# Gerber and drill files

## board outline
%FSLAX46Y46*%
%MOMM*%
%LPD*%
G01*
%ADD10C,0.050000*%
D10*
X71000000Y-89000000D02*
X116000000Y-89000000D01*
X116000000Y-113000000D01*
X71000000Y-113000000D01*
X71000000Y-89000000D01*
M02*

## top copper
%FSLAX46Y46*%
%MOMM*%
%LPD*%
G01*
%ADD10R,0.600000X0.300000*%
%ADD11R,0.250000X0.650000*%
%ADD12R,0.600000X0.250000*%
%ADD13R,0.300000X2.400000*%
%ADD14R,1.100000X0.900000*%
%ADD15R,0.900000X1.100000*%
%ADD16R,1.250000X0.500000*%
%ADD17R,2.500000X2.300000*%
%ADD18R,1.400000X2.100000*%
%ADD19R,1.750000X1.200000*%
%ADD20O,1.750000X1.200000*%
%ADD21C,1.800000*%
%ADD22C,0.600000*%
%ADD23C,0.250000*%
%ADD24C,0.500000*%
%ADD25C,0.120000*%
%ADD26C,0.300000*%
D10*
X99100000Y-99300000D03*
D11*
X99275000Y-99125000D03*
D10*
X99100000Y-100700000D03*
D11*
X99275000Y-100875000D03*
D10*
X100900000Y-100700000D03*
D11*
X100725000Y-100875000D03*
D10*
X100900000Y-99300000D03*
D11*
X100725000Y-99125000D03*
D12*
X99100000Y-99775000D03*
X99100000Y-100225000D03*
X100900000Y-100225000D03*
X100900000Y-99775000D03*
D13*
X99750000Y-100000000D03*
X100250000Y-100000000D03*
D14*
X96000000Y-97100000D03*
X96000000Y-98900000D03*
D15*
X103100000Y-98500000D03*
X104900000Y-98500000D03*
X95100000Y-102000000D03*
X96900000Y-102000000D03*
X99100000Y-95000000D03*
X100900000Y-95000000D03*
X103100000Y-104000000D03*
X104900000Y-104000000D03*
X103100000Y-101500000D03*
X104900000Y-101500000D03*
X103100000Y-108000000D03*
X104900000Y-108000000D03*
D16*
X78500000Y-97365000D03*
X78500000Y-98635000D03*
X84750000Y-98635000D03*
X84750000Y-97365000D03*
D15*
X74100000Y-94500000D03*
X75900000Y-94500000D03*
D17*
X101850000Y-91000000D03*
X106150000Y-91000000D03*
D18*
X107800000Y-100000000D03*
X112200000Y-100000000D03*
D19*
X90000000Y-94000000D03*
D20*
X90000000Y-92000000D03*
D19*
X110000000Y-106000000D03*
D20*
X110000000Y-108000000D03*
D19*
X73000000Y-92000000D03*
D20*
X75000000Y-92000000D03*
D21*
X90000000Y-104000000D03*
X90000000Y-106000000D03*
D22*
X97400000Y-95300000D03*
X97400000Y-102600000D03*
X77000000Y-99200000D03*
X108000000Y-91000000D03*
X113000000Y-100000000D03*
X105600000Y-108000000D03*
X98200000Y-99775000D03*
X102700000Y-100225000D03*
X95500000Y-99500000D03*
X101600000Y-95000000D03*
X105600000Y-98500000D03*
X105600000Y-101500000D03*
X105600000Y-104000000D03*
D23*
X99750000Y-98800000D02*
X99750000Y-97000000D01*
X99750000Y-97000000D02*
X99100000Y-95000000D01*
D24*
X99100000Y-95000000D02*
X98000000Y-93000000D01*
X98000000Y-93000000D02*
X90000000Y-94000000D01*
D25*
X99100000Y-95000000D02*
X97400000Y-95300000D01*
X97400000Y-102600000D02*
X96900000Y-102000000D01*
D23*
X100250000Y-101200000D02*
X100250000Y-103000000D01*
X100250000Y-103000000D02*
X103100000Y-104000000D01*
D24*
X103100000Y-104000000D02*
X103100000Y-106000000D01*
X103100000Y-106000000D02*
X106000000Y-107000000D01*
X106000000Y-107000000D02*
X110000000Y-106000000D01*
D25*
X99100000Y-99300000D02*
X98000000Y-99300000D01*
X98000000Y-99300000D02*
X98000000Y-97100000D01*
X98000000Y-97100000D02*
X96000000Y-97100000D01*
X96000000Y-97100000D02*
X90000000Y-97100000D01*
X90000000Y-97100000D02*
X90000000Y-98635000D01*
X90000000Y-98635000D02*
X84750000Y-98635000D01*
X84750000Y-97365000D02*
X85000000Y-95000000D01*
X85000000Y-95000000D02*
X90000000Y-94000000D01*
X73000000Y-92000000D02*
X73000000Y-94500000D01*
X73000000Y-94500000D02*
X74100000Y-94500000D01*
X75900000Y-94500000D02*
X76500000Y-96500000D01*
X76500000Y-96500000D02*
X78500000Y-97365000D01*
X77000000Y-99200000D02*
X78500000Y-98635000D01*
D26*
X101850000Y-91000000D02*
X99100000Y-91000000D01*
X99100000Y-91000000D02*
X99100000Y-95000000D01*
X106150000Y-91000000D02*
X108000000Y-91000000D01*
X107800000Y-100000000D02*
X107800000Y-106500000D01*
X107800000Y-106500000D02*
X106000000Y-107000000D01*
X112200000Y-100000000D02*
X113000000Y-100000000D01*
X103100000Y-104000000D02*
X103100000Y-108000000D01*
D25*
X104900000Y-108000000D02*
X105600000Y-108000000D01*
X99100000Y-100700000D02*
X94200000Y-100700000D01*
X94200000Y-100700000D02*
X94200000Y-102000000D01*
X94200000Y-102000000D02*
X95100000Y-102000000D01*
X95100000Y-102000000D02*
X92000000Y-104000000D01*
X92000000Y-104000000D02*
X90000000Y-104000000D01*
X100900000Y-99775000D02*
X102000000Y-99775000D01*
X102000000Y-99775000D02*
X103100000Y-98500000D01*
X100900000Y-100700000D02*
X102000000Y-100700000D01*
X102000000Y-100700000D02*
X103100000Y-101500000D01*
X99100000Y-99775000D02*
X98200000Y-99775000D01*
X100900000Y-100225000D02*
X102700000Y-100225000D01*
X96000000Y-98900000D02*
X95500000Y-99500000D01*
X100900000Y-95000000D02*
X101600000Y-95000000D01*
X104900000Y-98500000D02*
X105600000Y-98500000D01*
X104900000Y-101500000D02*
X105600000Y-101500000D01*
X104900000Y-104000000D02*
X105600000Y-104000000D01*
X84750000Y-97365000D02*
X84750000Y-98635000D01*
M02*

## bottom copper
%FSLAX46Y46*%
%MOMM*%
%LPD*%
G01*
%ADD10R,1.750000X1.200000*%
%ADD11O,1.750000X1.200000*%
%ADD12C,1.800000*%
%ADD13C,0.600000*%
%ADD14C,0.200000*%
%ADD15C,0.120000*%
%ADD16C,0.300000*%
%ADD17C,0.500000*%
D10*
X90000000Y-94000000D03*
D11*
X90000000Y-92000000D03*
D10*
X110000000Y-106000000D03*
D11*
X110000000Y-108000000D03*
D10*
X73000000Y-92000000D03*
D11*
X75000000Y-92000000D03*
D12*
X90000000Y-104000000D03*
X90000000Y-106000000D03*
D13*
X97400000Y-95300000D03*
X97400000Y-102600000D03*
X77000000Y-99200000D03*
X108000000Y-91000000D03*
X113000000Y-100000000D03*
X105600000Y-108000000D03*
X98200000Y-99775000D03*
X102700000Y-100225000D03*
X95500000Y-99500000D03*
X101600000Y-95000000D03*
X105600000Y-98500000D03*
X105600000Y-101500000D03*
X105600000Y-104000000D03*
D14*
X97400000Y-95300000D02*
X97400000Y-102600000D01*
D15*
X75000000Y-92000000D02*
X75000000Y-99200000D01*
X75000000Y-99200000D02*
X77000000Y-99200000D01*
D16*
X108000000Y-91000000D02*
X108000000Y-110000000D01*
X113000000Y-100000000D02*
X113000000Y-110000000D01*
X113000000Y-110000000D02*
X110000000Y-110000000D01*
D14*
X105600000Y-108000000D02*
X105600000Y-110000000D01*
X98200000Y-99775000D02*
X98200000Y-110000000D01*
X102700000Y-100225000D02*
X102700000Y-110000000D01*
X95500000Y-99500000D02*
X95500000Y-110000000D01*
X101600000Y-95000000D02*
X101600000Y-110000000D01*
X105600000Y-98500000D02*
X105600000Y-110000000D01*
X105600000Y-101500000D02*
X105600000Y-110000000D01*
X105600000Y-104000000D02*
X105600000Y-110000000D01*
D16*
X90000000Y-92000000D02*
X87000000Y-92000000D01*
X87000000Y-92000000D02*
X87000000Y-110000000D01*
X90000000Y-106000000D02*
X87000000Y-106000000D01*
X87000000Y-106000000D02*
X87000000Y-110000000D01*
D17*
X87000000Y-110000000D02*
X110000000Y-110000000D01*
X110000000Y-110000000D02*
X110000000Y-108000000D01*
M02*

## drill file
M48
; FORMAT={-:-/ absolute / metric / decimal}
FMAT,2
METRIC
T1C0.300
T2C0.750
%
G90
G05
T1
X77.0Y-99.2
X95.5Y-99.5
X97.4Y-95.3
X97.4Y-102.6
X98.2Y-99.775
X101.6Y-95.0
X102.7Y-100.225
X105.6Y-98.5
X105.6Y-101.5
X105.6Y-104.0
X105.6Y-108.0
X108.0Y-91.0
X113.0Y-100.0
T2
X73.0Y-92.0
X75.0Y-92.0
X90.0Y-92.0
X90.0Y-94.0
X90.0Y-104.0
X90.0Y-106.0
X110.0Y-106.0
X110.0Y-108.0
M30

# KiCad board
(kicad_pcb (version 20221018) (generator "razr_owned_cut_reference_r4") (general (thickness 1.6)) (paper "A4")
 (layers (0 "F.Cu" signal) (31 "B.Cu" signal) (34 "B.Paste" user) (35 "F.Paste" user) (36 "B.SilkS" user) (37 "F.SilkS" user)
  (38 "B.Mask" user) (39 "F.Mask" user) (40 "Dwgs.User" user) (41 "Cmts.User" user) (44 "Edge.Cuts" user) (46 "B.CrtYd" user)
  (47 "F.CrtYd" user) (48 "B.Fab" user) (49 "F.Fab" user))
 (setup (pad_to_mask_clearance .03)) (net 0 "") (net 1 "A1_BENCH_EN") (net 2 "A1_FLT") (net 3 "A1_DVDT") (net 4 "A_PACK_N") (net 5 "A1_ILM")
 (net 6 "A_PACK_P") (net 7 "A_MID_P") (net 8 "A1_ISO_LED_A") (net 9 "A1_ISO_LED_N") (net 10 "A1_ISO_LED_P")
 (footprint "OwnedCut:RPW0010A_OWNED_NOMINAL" (layer "F.Cu") (at 100 100)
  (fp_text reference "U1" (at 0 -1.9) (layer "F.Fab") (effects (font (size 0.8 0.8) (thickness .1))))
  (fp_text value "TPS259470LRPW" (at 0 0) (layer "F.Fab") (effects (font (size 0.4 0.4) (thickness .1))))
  (pad "1" smd rect (at -0.9 -0.7) (size 0.6 0.3) (layers "F.Cu" "F.Paste" "F.Mask") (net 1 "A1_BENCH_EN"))
  (pad "1" smd rect (at -0.725 -0.875) (size 0.25 0.65) (layers "F.Cu" "F.Paste" "F.Mask") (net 1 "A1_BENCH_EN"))
  (pad "4" smd rect (at -0.9 0.7) (size 0.6 0.3) (layers "F.Cu" "F.Paste" "F.Mask") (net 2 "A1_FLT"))
  (pad "4" smd rect (at -0.725 0.875) (size 0.25 0.65) (layers "F.Cu" "F.Paste" "F.Mask") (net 2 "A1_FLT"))
  (pad "7" smd rect (at 0.9 0.7) (size 0.6 0.3) (layers "F.Cu" "F.Paste" "F.Mask") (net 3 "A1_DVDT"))
  (pad "7" smd rect (at 0.725 0.875) (size 0.25 0.65) (layers "F.Cu" "F.Paste" "F.Mask") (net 3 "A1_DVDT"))
  (pad "10" smd rect (at 0.9 -0.7) (size 0.6 0.3) (layers "F.Cu" "F.Paste" "F.Mask"))
  (pad "10" smd rect (at 0.725 -0.875) (size 0.25 0.65) (layers "F.Cu" "F.Paste" "F.Mask"))
  (pad "2" smd rect (at -0.9 -0.225) (size 0.6 0.25) (layers "F.Cu" "F.Paste" "F.Mask") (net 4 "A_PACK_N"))
  (pad "3" smd rect (at -0.9 0.225) (size 0.6 0.25) (layers "F.Cu" "F.Paste" "F.Mask"))
  (pad "8" smd rect (at 0.9 0.225) (size 0.6 0.25) (layers "F.Cu" "F.Paste" "F.Mask") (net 4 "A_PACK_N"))
  (pad "9" smd rect (at 0.9 -0.225) (size 0.6 0.25) (layers "F.Cu" "F.Paste" "F.Mask") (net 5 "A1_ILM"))
  (pad "5" smd rect (at -0.25 0) (size 0.3 2.4) (layers "F.Cu" "F.Paste" "F.Mask") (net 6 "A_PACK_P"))
  (pad "6" smd rect (at 0.25 0) (size 0.3 2.4) (layers "F.Cu" "F.Paste" "F.Mask") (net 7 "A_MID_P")))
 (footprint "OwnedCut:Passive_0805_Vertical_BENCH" (layer "F.Cu") (at 96 98)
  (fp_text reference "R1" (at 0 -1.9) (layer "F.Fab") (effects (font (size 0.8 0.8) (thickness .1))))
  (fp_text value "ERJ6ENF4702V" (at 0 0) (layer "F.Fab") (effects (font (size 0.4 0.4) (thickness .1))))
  (pad "1" smd rect (at 0 -0.9) (size 1.1 0.9) (layers "F.Cu" "F.Paste" "F.Mask") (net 1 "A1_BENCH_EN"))
  (pad "2" smd rect (at 0 0.9) (size 1.1 0.9) (layers "F.Cu" "F.Paste" "F.Mask") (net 4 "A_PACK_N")))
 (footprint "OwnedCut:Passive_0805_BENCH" (layer "F.Cu") (at 104 98.5)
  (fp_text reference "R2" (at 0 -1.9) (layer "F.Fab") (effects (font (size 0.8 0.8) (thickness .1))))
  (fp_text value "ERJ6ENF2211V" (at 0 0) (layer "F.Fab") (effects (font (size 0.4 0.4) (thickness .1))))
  (pad "1" smd rect (at -0.9 0) (size 0.9 1.1) (layers "F.Cu" "F.Paste" "F.Mask") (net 5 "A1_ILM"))
  (pad "2" smd rect (at 0.9 0) (size 0.9 1.1) (layers "F.Cu" "F.Paste" "F.Mask") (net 4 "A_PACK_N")))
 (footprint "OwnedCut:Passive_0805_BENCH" (layer "F.Cu") (at 96 102)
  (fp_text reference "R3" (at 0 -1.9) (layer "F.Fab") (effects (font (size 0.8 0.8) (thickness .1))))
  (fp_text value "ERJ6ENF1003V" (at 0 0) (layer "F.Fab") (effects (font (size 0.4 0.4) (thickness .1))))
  (pad "1" smd rect (at -0.9 0) (size 0.9 1.1) (layers "F.Cu" "F.Paste" "F.Mask") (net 2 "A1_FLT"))
  (pad "2" smd rect (at 0.9 0) (size 0.9 1.1) (layers "F.Cu" "F.Paste" "F.Mask") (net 6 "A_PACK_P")))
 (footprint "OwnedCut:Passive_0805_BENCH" (layer "F.Cu") (at 100 95)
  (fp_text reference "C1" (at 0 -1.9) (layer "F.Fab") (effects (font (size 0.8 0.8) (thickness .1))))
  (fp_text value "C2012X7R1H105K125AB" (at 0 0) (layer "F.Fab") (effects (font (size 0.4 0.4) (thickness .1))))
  (pad "1" smd rect (at -0.9 0) (size 0.9 1.1) (layers "F.Cu" "F.Paste" "F.Mask") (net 6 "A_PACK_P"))
  (pad "2" smd rect (at 0.9 0) (size 0.9 1.1) (layers "F.Cu" "F.Paste" "F.Mask") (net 4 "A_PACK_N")))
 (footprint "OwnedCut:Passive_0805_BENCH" (layer "F.Cu") (at 104 104)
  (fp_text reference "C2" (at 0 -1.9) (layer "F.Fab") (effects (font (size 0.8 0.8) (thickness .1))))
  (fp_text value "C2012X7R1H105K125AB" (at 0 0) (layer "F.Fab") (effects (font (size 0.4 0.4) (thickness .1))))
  (pad "1" smd rect (at -0.9 0) (size 0.9 1.1) (layers "F.Cu" "F.Paste" "F.Mask") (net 7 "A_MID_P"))
  (pad "2" smd rect (at 0.9 0) (size 0.9 1.1) (layers "F.Cu" "F.Paste" "F.Mask") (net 4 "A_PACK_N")))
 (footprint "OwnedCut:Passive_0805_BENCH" (layer "F.Cu") (at 104 101.5)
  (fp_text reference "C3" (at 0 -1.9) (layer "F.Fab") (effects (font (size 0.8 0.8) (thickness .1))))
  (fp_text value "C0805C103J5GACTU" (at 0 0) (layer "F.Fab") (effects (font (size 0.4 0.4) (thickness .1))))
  (pad "1" smd rect (at -0.9 0) (size 0.9 1.1) (layers "F.Cu" "F.Paste" "F.Mask") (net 3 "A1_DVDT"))
  (pad "2" smd rect (at 0.9 0) (size 0.9 1.1) (layers "F.Cu" "F.Paste" "F.Mask") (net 4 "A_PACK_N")))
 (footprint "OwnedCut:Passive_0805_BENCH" (layer "F.Cu") (at 104 108)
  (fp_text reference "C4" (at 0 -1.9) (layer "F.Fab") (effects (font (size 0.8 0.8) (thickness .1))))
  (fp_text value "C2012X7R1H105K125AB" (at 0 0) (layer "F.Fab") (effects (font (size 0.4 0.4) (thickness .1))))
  (pad "1" smd rect (at -0.9 0) (size 0.9 1.1) (layers "F.Cu" "F.Paste" "F.Mask") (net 7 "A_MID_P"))
  (pad "2" smd rect (at 0.9 0) (size 0.9 1.1) (layers "F.Cu" "F.Paste" "F.Mask") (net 4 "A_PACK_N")))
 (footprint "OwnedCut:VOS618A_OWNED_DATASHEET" (layer "F.Cu") (at 81.625 98)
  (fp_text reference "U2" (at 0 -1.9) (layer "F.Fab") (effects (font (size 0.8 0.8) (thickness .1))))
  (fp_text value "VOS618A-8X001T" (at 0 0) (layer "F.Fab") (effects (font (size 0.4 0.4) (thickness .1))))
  (pad "1" smd rect (at -3.125 -0.635) (size 1.25 0.5) (layers "F.Cu" "F.Paste" "F.Mask") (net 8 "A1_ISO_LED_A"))
  (pad "2" smd rect (at -3.125 0.635) (size 1.25 0.5) (layers "F.Cu" "F.Paste" "F.Mask") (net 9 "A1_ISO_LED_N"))
  (pad "3" smd rect (at 3.125 0.635) (size 1.25 0.5) (layers "F.Cu" "F.Paste" "F.Mask") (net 1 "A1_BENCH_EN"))
  (pad "4" smd rect (at 3.125 -0.635) (size 1.25 0.5) (layers "F.Cu" "F.Paste" "F.Mask") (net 6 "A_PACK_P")))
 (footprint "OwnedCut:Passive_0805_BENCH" (layer "F.Cu") (at 75 94.5)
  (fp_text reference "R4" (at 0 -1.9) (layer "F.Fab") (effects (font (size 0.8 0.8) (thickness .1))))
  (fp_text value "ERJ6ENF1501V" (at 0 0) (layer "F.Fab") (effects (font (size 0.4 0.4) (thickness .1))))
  (pad "1" smd rect (at -0.9 0) (size 0.9 1.1) (layers "F.Cu" "F.Paste" "F.Mask") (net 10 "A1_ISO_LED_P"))
  (pad "2" smd rect (at 0.9 0) (size 0.9 1.1) (layers "F.Cu" "F.Paste" "F.Mask") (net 8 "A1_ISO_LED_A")))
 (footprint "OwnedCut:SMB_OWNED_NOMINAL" (layer "F.Cu") (at 104 91)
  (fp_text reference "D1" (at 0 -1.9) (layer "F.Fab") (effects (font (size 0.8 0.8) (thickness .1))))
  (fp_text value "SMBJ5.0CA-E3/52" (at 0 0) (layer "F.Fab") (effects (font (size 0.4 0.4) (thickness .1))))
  (pad "1" smd rect (at -2.15 0) (size 2.5 2.3) (layers "F.Cu" "F.Paste" "F.Mask") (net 6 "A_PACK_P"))
  (pad "2" smd rect (at 2.15 0) (size 2.5 2.3) (layers "F.Cu" "F.Paste" "F.Mask") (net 4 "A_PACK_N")))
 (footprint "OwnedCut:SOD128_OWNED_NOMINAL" (layer "F.Cu") (at 110 100)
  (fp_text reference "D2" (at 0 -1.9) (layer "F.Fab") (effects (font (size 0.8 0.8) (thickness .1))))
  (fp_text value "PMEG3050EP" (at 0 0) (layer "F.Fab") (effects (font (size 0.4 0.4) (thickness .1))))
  (pad "1" smd rect (at -2.2 0) (size 1.4 2.1) (layers "F.Cu" "F.Paste" "F.Mask") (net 7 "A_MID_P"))
  (pad "2" smd rect (at 2.2 0) (size 1.4 2.1) (layers "F.Cu" "F.Paste" "F.Mask") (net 4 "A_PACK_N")))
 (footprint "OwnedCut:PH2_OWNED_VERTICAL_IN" (layer "F.Cu") (at 90 94)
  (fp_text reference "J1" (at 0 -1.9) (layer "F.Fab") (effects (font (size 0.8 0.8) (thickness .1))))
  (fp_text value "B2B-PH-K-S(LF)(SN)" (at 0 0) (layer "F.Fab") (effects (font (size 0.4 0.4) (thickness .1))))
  (pad "1" thru_hole rect (at 0 0) (size 1.75 1.2) (drill .75) (layers "*.Cu" "*.Mask") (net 6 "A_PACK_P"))
  (pad "2" thru_hole oval (at 0 -2) (size 1.75 1.2) (drill .75) (layers "*.Cu" "*.Mask") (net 4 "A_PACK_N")))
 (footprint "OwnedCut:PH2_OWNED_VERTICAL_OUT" (layer "F.Cu") (at 110 106)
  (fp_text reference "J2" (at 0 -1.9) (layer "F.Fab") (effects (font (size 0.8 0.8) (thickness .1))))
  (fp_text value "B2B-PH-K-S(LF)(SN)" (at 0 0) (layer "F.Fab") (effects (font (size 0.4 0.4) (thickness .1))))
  (pad "1" thru_hole rect (at 0 0) (size 1.75 1.2) (drill .75) (layers "*.Cu" "*.Mask") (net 7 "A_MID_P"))
  (pad "2" thru_hole oval (at 0 2) (size 1.75 1.2) (drill .75) (layers "*.Cu" "*.Mask") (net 4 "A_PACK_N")))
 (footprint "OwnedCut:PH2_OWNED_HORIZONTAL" (layer "F.Cu") (at 73 92)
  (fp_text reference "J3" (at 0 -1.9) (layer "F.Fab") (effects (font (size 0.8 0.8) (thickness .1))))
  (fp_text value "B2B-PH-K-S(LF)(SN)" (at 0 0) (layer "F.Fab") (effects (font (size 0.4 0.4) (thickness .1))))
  (pad "1" thru_hole rect (at 0 0) (size 1.75 1.2) (drill .75) (layers "*.Cu" "*.Mask") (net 10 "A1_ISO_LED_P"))
  (pad "2" thru_hole oval (at 2 0) (size 1.75 1.2) (drill .75) (layers "*.Cu" "*.Mask") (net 9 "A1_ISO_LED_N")))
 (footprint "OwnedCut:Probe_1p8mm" (layer "F.Cu") (at 90 104)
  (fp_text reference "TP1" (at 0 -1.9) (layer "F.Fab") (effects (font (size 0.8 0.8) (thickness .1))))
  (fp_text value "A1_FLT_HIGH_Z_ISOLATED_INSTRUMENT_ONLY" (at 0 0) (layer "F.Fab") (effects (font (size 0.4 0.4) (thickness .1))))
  (pad "1" thru_hole circle (at 0 0) (size 1.8 1.8) (drill .75) (layers "*.Cu" "*.Mask") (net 2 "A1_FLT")))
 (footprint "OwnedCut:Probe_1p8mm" (layer "F.Cu") (at 90 106)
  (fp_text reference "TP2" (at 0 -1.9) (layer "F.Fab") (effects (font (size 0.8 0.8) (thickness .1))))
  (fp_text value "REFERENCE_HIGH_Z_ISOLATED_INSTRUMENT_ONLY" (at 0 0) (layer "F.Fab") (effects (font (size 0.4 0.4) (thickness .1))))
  (pad "1" thru_hole circle (at 0 0) (size 1.8 1.8) (drill .75) (layers "*.Cu" "*.Mask") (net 4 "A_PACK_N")))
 (segment (start 99.75 98.8) (end 99.75 97) (width 0.25) (layer "F.Cu") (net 6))
 (segment (start 99.75 97) (end 99.1 95) (width 0.25) (layer "F.Cu") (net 6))
 (segment (start 99.1 95) (end 98 93) (width 0.5) (layer "F.Cu") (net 6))
 (segment (start 98 93) (end 90 94) (width 0.5) (layer "F.Cu") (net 6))
 (segment (start 99.1 95) (end 97.4 95.3) (width 0.12) (layer "F.Cu") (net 6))
 (via (at 97.4 95.3) (size .6) (drill .3) (layers "F.Cu" "B.Cu") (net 6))
 (segment (start 97.4 95.3) (end 97.4 102.6) (width 0.2) (layer "B.Cu") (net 6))
 (via (at 97.4 102.6) (size .6) (drill .3) (layers "F.Cu" "B.Cu") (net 6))
 (segment (start 97.4 102.6) (end 96.9 102) (width 0.12) (layer "F.Cu") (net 6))
 (segment (start 100.25 101.2) (end 100.25 103) (width 0.25) (layer "F.Cu") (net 7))
 (segment (start 100.25 103) (end 103.1 104) (width 0.25) (layer "F.Cu") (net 7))
 (segment (start 103.1 104) (end 103.1 106) (width 0.5) (layer "F.Cu") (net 7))
 (segment (start 103.1 106) (end 106 107) (width 0.5) (layer "F.Cu") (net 7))
 (segment (start 106 107) (end 110 106) (width 0.5) (layer "F.Cu") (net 7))
 (segment (start 99.1 99.3) (end 98 99.3) (width 0.12) (layer "F.Cu") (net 1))
 (segment (start 98 99.3) (end 98 97.1) (width 0.12) (layer "F.Cu") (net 1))
 (segment (start 98 97.1) (end 96 97.1) (width 0.12) (layer "F.Cu") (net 1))
 (segment (start 96 97.1) (end 90 97.1) (width 0.12) (layer "F.Cu") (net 1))
 (segment (start 90 97.1) (end 90 98.635) (width 0.12) (layer "F.Cu") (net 1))
 (segment (start 90 98.635) (end 84.75 98.635) (width 0.12) (layer "F.Cu") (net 1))
 (segment (start 84.75 97.365) (end 85 95) (width 0.12) (layer "F.Cu") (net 6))
 (segment (start 85 95) (end 90 94) (width 0.12) (layer "F.Cu") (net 6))
 (segment (start 73 92) (end 73 94.5) (width 0.12) (layer "F.Cu") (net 10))
 (segment (start 73 94.5) (end 74.1 94.5) (width 0.12) (layer "F.Cu") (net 10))
 (segment (start 75.9 94.5) (end 76.5 96.5) (width 0.12) (layer "F.Cu") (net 8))
 (segment (start 76.5 96.5) (end 78.5 97.365) (width 0.12) (layer "F.Cu") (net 8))
 (segment (start 75 92) (end 75 99.2) (width 0.12) (layer "B.Cu") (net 9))
 (segment (start 75 99.2) (end 77 99.2) (width 0.12) (layer "B.Cu") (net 9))
 (via (at 77 99.2) (size .6) (drill .3) (layers "F.Cu" "B.Cu") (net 9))
 (segment (start 77 99.2) (end 78.5 98.635) (width 0.12) (layer "F.Cu") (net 9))
 (segment (start 101.85 91) (end 99.1 91) (width 0.3) (layer "F.Cu") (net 6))
 (segment (start 99.1 91) (end 99.1 95) (width 0.3) (layer "F.Cu") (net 6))
 (segment (start 106.15 91) (end 108 91) (width 0.3) (layer "F.Cu") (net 4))
 (via (at 108 91) (size .6) (drill .3) (layers "F.Cu" "B.Cu") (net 4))
 (segment (start 108 91) (end 108 110) (width 0.3) (layer "B.Cu") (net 4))
 (segment (start 107.8 100) (end 107.8 106.5) (width 0.3) (layer "F.Cu") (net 7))
 (segment (start 107.8 106.5) (end 106 107) (width 0.3) (layer "F.Cu") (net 7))
 (segment (start 112.2 100) (end 113 100) (width 0.3) (layer "F.Cu") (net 4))
 (via (at 113 100) (size .6) (drill .3) (layers "F.Cu" "B.Cu") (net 4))
 (segment (start 113 100) (end 113 110) (width 0.3) (layer "B.Cu") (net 4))
 (segment (start 113 110) (end 110 110) (width 0.3) (layer "B.Cu") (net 4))
 (segment (start 103.1 104) (end 103.1 108) (width 0.3) (layer "F.Cu") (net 7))
 (segment (start 104.9 108) (end 105.6 108) (width 0.12) (layer "F.Cu") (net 4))
 (via (at 105.6 108) (size .6) (drill .3) (layers "F.Cu" "B.Cu") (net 4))
 (segment (start 105.6 108) (end 105.6 110) (width 0.2) (layer "B.Cu") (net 4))
 (segment (start 99.1 100.7) (end 94.2 100.7) (width 0.12) (layer "F.Cu") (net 2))
 (segment (start 94.2 100.7) (end 94.2 102) (width 0.12) (layer "F.Cu") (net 2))
 (segment (start 94.2 102) (end 95.1 102) (width 0.12) (layer "F.Cu") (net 2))
 (segment (start 95.1 102) (end 92 104) (width 0.12) (layer "F.Cu") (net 2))
 (segment (start 92 104) (end 90 104) (width 0.12) (layer "F.Cu") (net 2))
 (segment (start 100.9 99.775) (end 102 99.775) (width 0.12) (layer "F.Cu") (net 5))
 (segment (start 102 99.775) (end 103.1 98.5) (width 0.12) (layer "F.Cu") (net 5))
 (segment (start 100.9 100.7) (end 102 100.7) (width 0.12) (layer "F.Cu") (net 3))
 (segment (start 102 100.7) (end 103.1 101.5) (width 0.12) (layer "F.Cu") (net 3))
 (segment (start 99.1 99.775) (end 98.2 99.775) (width 0.12) (layer "F.Cu") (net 4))
 (via (at 98.2 99.775) (size .6) (drill .3) (layers "F.Cu" "B.Cu") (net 4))
 (segment (start 98.2 99.775) (end 98.2 110) (width 0.2) (layer "B.Cu") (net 4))
 (segment (start 100.9 100.225) (end 102.7 100.225) (width 0.12) (layer "F.Cu") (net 4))
 (via (at 102.7 100.225) (size .6) (drill .3) (layers "F.Cu" "B.Cu") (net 4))
 (segment (start 102.7 100.225) (end 102.7 110) (width 0.2) (layer "B.Cu") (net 4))
 (segment (start 96 98.9) (end 95.5 99.5) (width 0.12) (layer "F.Cu") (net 4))
 (via (at 95.5 99.5) (size .6) (drill .3) (layers "F.Cu" "B.Cu") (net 4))
 (segment (start 95.5 99.5) (end 95.5 110) (width 0.2) (layer "B.Cu") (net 4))
 (segment (start 100.9 95) (end 101.6 95) (width 0.12) (layer "F.Cu") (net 4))
 (via (at 101.6 95) (size .6) (drill .3) (layers "F.Cu" "B.Cu") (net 4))
 (segment (start 101.6 95) (end 101.6 110) (width 0.2) (layer "B.Cu") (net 4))
 (segment (start 104.9 98.5) (end 105.6 98.5) (width 0.12) (layer "F.Cu") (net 4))
 (via (at 105.6 98.5) (size .6) (drill .3) (layers "F.Cu" "B.Cu") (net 4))
 (segment (start 105.6 98.5) (end 105.6 110) (width 0.2) (layer "B.Cu") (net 4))
 (segment (start 104.9 101.5) (end 105.6 101.5) (width 0.12) (layer "F.Cu") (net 4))
 (via (at 105.6 101.5) (size .6) (drill .3) (layers "F.Cu" "B.Cu") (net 4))
 (segment (start 105.6 101.5) (end 105.6 110) (width 0.2) (layer "B.Cu") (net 4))
 (segment (start 104.9 104) (end 105.6 104) (width 0.12) (layer "F.Cu") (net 4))
 (via (at 105.6 104) (size .6) (drill .3) (layers "F.Cu" "B.Cu") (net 4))
 (segment (start 105.6 104) (end 105.6 110) (width 0.2) (layer "B.Cu") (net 4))
 (segment (start 90 92) (end 87 92) (width 0.3) (layer "B.Cu") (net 4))
 (segment (start 87 92) (end 87 110) (width 0.3) (layer "B.Cu") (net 4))
 (segment (start 90 106) (end 87 106) (width 0.3) (layer "B.Cu") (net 4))
 (segment (start 87 106) (end 87 110) (width 0.3) (layer "B.Cu") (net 4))
 (segment (start 87 110) (end 110 110) (width 0.5) (layer "B.Cu") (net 4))
 (segment (start 110 110) (end 110 108) (width 0.5) (layer "B.Cu") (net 4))
 (gr_rect (start 71 89) (end 116 113) (stroke (width .05) (type default)) (fill none) (layer "Edge.Cuts"))
 (segment (start 84.75 97.365) (end 84.75 98.635) (width .12) (layer "F.Cu") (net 6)))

